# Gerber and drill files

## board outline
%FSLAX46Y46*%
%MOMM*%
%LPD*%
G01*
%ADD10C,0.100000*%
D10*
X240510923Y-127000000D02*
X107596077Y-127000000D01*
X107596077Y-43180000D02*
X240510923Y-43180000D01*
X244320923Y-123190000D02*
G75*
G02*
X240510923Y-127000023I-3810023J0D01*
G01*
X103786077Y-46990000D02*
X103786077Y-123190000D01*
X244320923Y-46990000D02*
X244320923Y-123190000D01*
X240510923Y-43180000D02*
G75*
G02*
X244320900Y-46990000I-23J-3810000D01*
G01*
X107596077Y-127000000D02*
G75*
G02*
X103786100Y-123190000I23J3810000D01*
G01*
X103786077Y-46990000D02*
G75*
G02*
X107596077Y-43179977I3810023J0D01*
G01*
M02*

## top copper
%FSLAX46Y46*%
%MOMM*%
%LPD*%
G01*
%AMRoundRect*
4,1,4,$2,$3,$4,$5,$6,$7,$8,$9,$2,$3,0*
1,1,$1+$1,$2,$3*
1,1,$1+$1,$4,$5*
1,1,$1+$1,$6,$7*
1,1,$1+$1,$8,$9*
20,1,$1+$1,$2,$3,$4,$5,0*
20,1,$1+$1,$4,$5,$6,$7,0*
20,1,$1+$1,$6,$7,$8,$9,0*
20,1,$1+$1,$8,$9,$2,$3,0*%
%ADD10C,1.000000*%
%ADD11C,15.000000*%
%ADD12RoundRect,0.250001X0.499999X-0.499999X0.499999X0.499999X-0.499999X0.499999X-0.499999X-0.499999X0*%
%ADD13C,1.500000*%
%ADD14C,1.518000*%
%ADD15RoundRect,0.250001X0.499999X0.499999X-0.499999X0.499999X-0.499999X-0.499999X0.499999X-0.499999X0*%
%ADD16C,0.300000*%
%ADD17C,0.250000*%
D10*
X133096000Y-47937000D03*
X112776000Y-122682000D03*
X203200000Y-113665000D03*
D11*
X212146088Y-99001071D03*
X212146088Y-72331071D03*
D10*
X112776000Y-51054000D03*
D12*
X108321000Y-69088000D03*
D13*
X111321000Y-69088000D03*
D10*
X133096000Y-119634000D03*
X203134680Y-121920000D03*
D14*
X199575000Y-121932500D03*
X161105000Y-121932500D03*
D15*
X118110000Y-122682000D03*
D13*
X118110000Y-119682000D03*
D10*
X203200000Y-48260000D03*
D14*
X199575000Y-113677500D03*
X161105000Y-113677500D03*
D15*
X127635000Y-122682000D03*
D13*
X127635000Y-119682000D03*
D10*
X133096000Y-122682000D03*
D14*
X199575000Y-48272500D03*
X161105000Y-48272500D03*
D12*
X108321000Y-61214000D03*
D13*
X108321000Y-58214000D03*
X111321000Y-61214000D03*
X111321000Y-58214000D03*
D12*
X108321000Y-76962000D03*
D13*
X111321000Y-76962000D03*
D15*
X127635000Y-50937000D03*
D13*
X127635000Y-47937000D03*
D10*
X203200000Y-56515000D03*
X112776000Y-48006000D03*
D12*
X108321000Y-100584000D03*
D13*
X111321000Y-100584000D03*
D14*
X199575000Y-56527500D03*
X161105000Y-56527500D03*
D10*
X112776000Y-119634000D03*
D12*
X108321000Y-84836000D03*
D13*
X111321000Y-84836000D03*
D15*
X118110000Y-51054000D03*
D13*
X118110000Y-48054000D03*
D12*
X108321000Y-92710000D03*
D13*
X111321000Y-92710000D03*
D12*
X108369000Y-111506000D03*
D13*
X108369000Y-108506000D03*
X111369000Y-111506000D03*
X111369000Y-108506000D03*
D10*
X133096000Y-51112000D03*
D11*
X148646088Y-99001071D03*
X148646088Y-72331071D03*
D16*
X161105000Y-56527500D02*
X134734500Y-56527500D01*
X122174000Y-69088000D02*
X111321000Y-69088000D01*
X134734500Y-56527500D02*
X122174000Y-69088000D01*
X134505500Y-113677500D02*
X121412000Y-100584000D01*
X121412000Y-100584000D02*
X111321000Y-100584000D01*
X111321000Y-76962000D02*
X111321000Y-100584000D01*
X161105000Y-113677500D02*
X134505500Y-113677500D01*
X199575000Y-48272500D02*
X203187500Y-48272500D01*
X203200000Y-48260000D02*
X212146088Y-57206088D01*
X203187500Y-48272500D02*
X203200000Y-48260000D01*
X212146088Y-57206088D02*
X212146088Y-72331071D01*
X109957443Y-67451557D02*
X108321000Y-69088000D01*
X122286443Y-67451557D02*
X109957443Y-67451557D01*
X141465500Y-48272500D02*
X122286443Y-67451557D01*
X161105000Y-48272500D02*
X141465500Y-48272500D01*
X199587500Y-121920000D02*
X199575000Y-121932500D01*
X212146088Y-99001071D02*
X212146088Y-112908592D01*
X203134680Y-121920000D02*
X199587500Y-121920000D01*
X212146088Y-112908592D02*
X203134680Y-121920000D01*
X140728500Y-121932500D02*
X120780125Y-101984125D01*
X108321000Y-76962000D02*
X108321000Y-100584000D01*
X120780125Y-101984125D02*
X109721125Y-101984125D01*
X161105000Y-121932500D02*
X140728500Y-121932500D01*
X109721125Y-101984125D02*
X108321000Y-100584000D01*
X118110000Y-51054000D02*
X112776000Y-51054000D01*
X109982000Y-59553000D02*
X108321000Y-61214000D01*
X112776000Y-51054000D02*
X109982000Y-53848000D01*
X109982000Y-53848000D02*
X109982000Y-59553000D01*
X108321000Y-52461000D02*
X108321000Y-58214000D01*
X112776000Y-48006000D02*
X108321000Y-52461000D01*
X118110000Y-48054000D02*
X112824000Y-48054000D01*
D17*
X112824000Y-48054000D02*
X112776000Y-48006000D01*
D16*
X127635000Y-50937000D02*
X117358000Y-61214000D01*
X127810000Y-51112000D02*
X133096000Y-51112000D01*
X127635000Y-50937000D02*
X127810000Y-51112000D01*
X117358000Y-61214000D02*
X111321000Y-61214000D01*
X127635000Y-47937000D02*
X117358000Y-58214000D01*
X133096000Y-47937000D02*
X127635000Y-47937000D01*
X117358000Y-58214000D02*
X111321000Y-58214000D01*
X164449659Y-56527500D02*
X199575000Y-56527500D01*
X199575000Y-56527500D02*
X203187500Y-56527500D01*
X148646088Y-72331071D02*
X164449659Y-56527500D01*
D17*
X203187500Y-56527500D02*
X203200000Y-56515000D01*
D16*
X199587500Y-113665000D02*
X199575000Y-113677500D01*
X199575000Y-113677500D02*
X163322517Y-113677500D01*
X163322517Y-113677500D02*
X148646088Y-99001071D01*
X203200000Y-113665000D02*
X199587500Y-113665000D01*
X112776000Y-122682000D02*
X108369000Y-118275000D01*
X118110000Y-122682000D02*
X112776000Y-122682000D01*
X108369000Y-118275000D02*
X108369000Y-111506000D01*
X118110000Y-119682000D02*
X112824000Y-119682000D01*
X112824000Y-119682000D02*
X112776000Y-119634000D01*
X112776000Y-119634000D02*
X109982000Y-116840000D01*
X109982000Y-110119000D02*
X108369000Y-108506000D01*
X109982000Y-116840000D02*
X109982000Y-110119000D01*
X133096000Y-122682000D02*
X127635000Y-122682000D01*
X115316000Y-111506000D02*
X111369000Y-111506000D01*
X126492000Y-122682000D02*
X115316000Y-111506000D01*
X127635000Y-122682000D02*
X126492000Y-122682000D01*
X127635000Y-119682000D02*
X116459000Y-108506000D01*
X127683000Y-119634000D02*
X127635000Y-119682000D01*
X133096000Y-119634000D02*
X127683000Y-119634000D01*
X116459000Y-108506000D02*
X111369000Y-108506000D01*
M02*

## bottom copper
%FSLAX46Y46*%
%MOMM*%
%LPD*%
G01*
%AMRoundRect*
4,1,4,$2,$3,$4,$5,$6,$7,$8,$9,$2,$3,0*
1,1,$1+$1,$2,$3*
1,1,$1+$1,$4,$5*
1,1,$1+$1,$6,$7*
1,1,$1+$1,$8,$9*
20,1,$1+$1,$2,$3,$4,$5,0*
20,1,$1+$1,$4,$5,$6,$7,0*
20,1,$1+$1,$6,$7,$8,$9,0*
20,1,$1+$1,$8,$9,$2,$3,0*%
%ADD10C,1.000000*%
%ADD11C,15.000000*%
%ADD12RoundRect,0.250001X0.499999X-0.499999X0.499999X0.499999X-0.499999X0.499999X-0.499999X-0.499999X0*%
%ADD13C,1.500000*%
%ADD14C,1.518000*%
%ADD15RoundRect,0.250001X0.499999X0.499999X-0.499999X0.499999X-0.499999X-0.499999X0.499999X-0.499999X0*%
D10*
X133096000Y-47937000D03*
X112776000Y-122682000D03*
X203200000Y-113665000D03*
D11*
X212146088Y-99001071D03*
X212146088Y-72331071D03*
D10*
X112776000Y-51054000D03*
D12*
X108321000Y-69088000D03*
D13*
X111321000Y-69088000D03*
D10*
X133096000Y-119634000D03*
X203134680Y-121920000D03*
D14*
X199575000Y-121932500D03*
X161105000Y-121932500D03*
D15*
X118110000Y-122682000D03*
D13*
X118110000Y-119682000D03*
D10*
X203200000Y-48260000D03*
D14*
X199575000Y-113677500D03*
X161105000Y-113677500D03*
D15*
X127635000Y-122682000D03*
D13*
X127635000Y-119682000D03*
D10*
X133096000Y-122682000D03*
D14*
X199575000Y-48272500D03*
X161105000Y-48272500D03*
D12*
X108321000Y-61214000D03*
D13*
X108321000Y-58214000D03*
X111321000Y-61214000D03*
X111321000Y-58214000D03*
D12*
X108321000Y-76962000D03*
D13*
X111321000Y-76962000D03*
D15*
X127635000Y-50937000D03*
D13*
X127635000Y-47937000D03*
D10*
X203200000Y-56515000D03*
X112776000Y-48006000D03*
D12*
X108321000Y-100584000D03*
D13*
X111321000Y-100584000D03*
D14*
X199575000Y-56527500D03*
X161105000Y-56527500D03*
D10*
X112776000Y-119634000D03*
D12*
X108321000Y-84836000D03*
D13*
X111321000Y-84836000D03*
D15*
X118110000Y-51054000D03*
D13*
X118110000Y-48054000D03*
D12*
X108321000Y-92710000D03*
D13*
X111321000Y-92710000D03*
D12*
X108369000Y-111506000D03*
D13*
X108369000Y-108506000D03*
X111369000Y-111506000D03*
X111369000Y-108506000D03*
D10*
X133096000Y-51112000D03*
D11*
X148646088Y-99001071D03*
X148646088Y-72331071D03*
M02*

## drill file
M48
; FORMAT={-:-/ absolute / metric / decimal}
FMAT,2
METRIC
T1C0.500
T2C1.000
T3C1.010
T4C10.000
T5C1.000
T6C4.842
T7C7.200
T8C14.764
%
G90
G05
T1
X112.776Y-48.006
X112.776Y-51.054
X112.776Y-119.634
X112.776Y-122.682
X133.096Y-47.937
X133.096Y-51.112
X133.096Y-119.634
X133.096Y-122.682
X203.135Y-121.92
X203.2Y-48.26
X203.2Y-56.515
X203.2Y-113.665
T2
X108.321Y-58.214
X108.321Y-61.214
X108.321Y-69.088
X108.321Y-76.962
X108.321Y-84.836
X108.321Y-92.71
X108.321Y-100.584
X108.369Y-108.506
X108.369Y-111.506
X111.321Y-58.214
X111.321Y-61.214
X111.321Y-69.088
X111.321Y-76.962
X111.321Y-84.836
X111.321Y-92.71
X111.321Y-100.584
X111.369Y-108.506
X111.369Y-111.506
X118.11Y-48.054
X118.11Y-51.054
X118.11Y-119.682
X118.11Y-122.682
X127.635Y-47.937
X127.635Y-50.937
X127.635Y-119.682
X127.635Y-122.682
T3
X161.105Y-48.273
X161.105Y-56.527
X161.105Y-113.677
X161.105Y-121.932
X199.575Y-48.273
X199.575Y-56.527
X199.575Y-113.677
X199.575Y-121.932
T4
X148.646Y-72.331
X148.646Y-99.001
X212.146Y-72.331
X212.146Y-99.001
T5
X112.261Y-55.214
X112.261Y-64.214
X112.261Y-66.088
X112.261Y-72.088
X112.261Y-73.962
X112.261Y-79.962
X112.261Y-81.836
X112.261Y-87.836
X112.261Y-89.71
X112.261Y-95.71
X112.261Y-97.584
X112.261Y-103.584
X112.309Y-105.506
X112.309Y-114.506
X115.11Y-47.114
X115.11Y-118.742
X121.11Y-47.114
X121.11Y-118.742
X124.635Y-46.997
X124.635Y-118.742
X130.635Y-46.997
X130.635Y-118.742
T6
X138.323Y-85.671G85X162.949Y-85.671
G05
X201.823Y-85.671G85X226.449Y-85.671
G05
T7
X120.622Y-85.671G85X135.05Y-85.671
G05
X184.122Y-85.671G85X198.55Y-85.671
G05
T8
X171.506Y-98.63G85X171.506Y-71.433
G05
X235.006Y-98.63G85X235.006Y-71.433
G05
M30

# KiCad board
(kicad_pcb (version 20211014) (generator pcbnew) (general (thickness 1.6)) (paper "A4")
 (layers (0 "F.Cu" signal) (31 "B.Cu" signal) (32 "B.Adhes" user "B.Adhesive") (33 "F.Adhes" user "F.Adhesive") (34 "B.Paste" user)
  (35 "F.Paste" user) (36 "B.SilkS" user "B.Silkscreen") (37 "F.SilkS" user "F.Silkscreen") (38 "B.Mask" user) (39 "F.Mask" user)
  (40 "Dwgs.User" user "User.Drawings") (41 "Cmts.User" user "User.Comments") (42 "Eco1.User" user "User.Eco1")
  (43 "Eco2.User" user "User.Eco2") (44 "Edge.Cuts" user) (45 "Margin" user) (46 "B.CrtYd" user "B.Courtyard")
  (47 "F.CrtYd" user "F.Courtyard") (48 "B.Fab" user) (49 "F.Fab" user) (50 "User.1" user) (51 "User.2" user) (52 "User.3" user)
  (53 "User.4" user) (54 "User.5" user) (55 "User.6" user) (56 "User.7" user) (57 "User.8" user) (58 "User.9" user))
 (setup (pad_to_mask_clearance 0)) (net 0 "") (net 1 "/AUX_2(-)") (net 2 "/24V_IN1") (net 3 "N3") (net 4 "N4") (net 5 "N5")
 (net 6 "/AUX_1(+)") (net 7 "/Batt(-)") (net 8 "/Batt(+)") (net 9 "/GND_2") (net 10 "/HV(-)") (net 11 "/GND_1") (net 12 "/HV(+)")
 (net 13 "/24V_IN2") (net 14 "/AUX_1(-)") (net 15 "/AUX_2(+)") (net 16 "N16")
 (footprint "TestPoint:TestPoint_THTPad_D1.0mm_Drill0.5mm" (layer "F.Cu") (at 133.096 47.937)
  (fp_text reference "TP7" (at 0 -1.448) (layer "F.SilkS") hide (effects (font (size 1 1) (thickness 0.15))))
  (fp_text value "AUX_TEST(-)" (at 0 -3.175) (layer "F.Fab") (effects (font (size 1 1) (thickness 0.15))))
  (pad "1" thru_hole circle (at 0 0) (size 1 1) (drill 0.5) (layers *.Cu *.Mask) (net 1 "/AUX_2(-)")))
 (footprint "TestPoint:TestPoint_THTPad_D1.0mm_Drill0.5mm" (layer "F.Cu") (at 112.776 122.682)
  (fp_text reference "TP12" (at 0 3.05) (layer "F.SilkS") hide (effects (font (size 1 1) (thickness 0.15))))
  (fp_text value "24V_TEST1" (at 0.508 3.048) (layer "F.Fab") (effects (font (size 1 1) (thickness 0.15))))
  (pad "1" thru_hole circle (at 0 0) (size 1 1) (drill 0.5) (layers *.Cu *.Mask) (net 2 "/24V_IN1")))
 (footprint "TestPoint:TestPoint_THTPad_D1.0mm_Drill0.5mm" (layer "F.Cu") (at 203.2 113.665)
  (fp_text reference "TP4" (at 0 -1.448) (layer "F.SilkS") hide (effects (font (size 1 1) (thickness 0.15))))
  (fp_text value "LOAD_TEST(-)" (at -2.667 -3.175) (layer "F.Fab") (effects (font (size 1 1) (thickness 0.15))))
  (pad "1" thru_hole circle (at 0 0) (size 1 1) (drill 0.5) (layers *.Cu *.Mask) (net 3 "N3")))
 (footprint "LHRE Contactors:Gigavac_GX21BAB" (layer "F.Cu") (at 182.738388 125.790071 90)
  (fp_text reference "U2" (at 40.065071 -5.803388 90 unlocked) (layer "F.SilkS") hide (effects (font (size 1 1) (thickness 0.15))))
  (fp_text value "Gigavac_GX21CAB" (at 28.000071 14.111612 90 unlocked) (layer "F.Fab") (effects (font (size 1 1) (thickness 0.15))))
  (pad "" np_thru_hole oval (at 40.119 31.3977 90) (size 4.84155 29.467172) (drill oval 4.84155 29.467172) (layers F&B.Cu *.Mask))
  (pad "" np_thru_hole oval (at 40.759 52.2677 90) (size 41.9608 14.76375) (drill oval 41.9608 14.76375) (layers F&B.Cu *.Mask))
  (pad "" np_thru_hole oval (at 40.119 8.5977 90) (size 7.2 21.6281) (drill oval 7.2 21.6281) (layers F&B.Cu *.Mask))
  (pad "1" thru_hole circle (at 26.789 29.4077 90) (size 15 15) (drill 10) (layers *.Cu *.Mask) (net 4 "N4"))
  (pad "2" thru_hole circle (at 53.459 29.4077 90) (size 15 15) (drill 10) (layers *.Cu *.Mask) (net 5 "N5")))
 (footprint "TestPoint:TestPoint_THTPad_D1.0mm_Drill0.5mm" (layer "F.Cu") (at 112.776 51.054)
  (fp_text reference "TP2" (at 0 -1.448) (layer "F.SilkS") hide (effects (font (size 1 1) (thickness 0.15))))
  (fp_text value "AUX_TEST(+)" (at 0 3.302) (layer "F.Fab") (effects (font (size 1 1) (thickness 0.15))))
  (pad "1" thru_hole circle (at 0 0) (size 1 1) (drill 0.5) (layers *.Cu *.Mask) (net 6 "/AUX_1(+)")))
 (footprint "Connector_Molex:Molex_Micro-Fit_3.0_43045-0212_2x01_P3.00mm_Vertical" (layer "F.Cu") (at 108.321 69.088 90)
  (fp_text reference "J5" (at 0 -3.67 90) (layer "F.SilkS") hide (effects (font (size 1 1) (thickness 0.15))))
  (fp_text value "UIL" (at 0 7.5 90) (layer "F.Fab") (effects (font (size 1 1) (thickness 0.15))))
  (pad "" np_thru_hole circle (at 3 3.94 90) (size 1 1) (drill 1) (layers *.Cu *.Mask))
  (pad "" np_thru_hole circle (at -3 3.94 90) (size 1 1) (drill 1) (layers *.Cu *.Mask))
  (pad "1" thru_hole roundrect (at 0 0 90) (size 1.5 1.5) (drill 1) (layers *.Cu *.Mask) (roundrect_rratio 0.166667) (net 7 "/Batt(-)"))
  (pad "2" thru_hole circle (at 0 3 90) (size 1.5 1.5) (drill 1) (layers *.Cu *.Mask) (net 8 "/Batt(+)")))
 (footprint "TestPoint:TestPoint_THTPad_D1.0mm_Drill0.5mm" (layer "F.Cu") (at 133.096 119.634)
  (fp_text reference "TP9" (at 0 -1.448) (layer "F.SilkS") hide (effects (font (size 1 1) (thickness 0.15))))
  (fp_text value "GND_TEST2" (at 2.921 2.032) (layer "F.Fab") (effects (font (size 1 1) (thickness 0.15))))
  (pad "1" thru_hole circle (at 0 0) (size 1 1) (drill 0.5) (layers *.Cu *.Mask) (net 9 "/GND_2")))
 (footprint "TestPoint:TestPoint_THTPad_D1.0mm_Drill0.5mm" (layer "F.Cu") (at 203.13468 121.92)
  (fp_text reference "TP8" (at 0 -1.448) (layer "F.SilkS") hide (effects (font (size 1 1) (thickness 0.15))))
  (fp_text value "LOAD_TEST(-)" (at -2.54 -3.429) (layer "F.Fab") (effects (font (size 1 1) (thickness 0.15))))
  (pad "1" thru_hole circle (at 0 0) (size 1 1) (drill 0.5) (layers *.Cu *.Mask) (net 4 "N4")))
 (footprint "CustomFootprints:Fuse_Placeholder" (layer "F.Cu") (at 180.44 129.1225 180)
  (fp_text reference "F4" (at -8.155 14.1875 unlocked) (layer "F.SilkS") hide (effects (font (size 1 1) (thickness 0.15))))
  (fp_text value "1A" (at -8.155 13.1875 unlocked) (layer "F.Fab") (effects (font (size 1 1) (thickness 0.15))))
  (pad "1" thru_hole circle (at -19.135 7.19 180) (size 1.518 1.518) (drill 1.01) (layers *.Cu *.Mask) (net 4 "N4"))
  (pad "2" thru_hole circle (at 19.335 7.19 180) (size 1.518 1.518) (drill 1.01) (layers *.Cu *.Mask) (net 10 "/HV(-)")))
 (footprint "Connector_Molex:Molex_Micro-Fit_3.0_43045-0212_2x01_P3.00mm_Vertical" (layer "F.Cu") (at 118.11 122.682 180)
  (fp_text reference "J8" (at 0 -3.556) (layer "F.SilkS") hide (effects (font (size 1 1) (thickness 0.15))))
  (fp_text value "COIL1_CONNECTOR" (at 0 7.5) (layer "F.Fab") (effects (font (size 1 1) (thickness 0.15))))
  (pad "" np_thru_hole circle (at -3 3.94 180) (size 1 1) (drill 1) (layers *.Cu *.Mask))
  (pad "" np_thru_hole circle (at 3 3.94 180) (size 1 1) (drill 1) (layers *.Cu *.Mask))
  (pad "1" thru_hole roundrect (at 0 0 180) (size 1.5 1.5) (drill 1) (layers *.Cu *.Mask) (roundrect_rratio 0.166667) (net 2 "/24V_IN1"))
  (pad "2" thru_hole circle (at 0 3 180) (size 1.5 1.5) (drill 1) (layers *.Cu *.Mask) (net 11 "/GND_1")))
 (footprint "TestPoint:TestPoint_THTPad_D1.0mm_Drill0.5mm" (layer "F.Cu") (at 203.2 48.26)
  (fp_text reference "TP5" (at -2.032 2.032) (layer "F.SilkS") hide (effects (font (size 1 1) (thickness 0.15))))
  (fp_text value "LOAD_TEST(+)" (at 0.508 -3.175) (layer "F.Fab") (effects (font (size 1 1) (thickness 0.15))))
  (pad "1" thru_hole circle (at 0 0) (size 1 1) (drill 0.5) (layers *.Cu *.Mask) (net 5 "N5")))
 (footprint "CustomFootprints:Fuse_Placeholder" (layer "F.Cu") (at 180.44 120.8675 180)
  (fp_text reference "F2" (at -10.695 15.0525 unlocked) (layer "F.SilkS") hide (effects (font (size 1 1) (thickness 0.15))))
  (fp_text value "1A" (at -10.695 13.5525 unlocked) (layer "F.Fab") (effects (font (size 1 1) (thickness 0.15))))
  (pad "1" thru_hole circle (at -19.135 7.19 180) (size 1.518 1.518) (drill 1.01) (layers *.Cu *.Mask) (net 3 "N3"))
  (pad "2" thru_hole circle (at 19.335 7.19 180) (size 1.518 1.518) (drill 1.01) (layers *.Cu *.Mask) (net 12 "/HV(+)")))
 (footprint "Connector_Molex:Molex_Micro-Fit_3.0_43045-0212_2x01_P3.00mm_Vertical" (layer "F.Cu") (at 127.635 122.682 180)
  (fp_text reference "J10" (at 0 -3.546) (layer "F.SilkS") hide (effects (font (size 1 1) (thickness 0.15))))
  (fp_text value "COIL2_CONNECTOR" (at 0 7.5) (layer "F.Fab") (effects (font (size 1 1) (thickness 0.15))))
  (pad "" np_thru_hole circle (at -3 3.94 180) (size 1 1) (drill 1) (layers *.Cu *.Mask))
  (pad "" np_thru_hole circle (at 3 3.94 180) (size 1 1) (drill 1) (layers *.Cu *.Mask))
  (pad "1" thru_hole roundrect (at 0 0 180) (size 1.5 1.5) (drill 1) (layers *.Cu *.Mask) (roundrect_rratio 0.166667) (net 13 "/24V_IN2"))
  (pad "2" thru_hole circle (at 0 3 180) (size 1.5 1.5) (drill 1) (layers *.Cu *.Mask) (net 9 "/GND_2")))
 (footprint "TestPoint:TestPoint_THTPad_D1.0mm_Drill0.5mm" (layer "F.Cu") (at 133.096 122.682)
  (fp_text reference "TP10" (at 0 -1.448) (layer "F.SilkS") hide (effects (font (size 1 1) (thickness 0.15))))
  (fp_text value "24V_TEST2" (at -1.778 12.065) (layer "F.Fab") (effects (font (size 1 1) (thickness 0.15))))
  (pad "1" thru_hole circle (at 0 0) (size 1 1) (drill 0.5) (layers *.Cu *.Mask) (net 13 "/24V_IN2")))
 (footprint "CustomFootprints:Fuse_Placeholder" (layer "F.Cu") (at 180.44 55.4625 180)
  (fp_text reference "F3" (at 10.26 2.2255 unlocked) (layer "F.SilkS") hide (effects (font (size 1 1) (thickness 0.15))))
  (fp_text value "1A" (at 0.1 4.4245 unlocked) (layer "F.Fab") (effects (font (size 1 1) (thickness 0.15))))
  (pad "1" thru_hole circle (at -19.135 7.19 180) (size 1.518 1.518) (drill 1.01) (layers *.Cu *.Mask) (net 5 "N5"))
  (pad "2" thru_hole circle (at 19.335 7.19 180) (size 1.518 1.518) (drill 1.01) (layers *.Cu *.Mask) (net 7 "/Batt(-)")))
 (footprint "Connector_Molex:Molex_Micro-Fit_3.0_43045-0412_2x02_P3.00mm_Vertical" (layer "F.Cu") (at 108.321 61.214 90)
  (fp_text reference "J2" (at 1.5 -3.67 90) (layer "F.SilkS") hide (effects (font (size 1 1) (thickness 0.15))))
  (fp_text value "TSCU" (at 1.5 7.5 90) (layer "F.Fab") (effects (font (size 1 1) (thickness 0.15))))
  (pad "" np_thru_hole circle (at -3 3.94 90) (size 1 1) (drill 1) (layers *.Cu *.Mask))
  (pad "" np_thru_hole circle (at 6 3.94 90) (size 1 1) (drill 1) (layers *.Cu *.Mask))
  (pad "1" thru_hole roundrect (at 0 0 90) (size 1.5 1.5) (drill 1) (layers *.Cu *.Mask) (roundrect_rratio 0.166667) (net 6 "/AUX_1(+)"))
  (pad "2" thru_hole circle (at 3 0 90) (size 1.5 1.5) (drill 1) (layers *.Cu *.Mask) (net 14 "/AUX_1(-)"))
  (pad "3" thru_hole circle (at 0 3 90) (size 1.5 1.5) (drill 1) (layers *.Cu *.Mask) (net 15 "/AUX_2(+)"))
  (pad "4" thru_hole circle (at 3 3 90) (size 1.5 1.5) (drill 1) (layers *.Cu *.Mask) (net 1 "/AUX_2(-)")))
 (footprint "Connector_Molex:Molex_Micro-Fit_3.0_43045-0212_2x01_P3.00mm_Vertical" (layer "F.Cu") (at 108.321 76.962 90)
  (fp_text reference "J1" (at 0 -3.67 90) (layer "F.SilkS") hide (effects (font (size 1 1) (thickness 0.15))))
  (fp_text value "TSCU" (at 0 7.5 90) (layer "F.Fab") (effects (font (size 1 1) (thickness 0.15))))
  (pad "" np_thru_hole circle (at 3 3.94 90) (size 1 1) (drill 1) (layers *.Cu *.Mask))
  (pad "" np_thru_hole circle (at -3 3.94 90) (size 1 1) (drill 1) (layers *.Cu *.Mask))
  (pad "1" thru_hole roundrect (at 0 0 90) (size 1.5 1.5) (drill 1) (layers *.Cu *.Mask) (roundrect_rratio 0.166667) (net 10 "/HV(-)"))
  (pad "2" thru_hole circle (at 0 3 90) (size 1.5 1.5) (drill 1) (layers *.Cu *.Mask) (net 12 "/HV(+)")))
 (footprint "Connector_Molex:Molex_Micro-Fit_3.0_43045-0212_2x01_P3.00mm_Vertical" (layer "F.Cu") (at 127.635 50.937 180)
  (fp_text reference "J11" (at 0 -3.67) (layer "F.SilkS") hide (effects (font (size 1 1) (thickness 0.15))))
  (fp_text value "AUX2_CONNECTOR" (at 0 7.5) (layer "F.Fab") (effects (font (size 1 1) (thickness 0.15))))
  (pad "" np_thru_hole circle (at 3 3.94 180) (size 1 1) (drill 1) (layers *.Cu *.Mask))
  (pad "" np_thru_hole circle (at -3 3.94 180) (size 1 1) (drill 1) (layers *.Cu *.Mask))
  (pad "1" thru_hole roundrect (at 0 0 180) (size 1.5 1.5) (drill 1) (layers *.Cu *.Mask) (roundrect_rratio 0.166667) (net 15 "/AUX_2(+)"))
  (pad "2" thru_hole circle (at 0 3 180) (size 1.5 1.5) (drill 1) (layers *.Cu *.Mask) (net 1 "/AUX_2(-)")))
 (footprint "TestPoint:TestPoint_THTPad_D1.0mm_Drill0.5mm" (layer "F.Cu") (at 203.2 56.515)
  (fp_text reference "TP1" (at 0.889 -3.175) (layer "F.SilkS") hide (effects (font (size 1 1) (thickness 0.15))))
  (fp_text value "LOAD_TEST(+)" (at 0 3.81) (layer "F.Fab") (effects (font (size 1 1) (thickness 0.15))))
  (pad "1" thru_hole circle (at 0 0) (size 1 1) (drill 0.5) (layers *.Cu *.Mask) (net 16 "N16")))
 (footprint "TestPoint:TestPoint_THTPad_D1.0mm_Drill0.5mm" (layer "F.Cu") (at 112.776 48.006)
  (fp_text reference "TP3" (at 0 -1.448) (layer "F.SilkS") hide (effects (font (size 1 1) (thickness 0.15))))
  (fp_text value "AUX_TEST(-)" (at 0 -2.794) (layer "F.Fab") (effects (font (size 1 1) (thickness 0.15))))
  (pad "1" thru_hole circle (at 0 0) (size 1 1) (drill 0.5) (layers *.Cu *.Mask) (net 14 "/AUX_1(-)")))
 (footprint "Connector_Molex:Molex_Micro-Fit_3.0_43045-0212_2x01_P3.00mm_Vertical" (layer "F.Cu") (at 108.321 100.584 90)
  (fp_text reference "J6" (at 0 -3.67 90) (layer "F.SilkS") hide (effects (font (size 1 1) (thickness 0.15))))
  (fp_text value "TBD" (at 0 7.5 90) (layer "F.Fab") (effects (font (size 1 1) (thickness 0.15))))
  (pad "" np_thru_hole circle (at 3 3.94 90) (size 1 1) (drill 1) (layers *.Cu *.Mask))
  (pad "" np_thru_hole circle (at -3 3.94 90) (size 1 1) (drill 1) (layers *.Cu *.Mask))
  (pad "1" thru_hole roundrect (at 0 0 90) (size 1.5 1.5) (drill 1) (layers *.Cu *.Mask) (roundrect_rratio 0.166667) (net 10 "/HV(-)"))
  (pad "2" thru_hole circle (at 0 3 90) (size 1.5 1.5) (drill 1) (layers *.Cu *.Mask) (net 12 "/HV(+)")))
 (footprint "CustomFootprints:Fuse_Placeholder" (layer "F.Cu") (at 180.44 63.7175 180)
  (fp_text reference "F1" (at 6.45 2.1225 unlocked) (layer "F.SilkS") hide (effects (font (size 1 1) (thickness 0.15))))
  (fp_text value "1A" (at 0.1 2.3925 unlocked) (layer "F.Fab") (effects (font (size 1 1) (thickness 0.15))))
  (pad "1" thru_hole circle (at -19.135 7.19 180) (size 1.518 1.518) (drill 1.01) (layers *.Cu *.Mask) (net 16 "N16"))
  (pad "2" thru_hole circle (at 19.335 7.19 180) (size 1.518 1.518) (drill 1.01) (layers *.Cu *.Mask) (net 8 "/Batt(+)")))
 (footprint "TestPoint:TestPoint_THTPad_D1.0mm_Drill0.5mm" (layer "F.Cu") (at 112.776 119.634)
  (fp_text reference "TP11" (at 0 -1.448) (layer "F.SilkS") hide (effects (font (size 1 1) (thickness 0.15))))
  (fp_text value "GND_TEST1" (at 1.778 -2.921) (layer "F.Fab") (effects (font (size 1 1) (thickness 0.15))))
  (pad "1" thru_hole circle (at 0 0) (size 1 1) (drill 0.5) (layers *.Cu *.Mask) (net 11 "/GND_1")))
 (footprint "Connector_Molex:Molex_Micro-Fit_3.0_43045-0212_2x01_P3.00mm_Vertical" (layer "F.Cu") (at 108.321 84.836 90)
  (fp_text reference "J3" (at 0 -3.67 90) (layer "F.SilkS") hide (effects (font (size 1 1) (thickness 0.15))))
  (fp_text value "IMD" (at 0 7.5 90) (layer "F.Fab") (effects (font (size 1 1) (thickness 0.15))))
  (pad "" np_thru_hole circle (at 3 3.94 90) (size 1 1) (drill 1) (layers *.Cu *.Mask))
  (pad "" np_thru_hole circle (at -3 3.94 90) (size 1 1) (drill 1) (layers *.Cu *.Mask))
  (pad "1" thru_hole roundrect (at 0 0 90) (size 1.5 1.5) (drill 1) (layers *.Cu *.Mask) (roundrect_rratio 0.166667) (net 10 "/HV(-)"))
  (pad "2" thru_hole circle (at 0 3 90) (size 1.5 1.5) (drill 1) (layers *.Cu *.Mask) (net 12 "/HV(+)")))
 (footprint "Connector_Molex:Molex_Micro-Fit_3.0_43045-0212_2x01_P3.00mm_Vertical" (layer "F.Cu") (at 118.11 51.054 180)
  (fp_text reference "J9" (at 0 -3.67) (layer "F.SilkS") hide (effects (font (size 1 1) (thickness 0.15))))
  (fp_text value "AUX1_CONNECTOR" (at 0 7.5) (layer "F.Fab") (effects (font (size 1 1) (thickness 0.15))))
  (pad "" np_thru_hole circle (at 3 3.94 180) (size 1 1) (drill 1) (layers *.Cu *.Mask))
  (pad "" np_thru_hole circle (at -3 3.94 180) (size 1 1) (drill 1) (layers *.Cu *.Mask))
  (pad "1" thru_hole roundrect (at 0 0 180) (size 1.5 1.5) (drill 1) (layers *.Cu *.Mask) (roundrect_rratio 0.166667) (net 6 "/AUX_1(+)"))
  (pad "2" thru_hole circle (at 0 3 180) (size 1.5 1.5) (drill 1) (layers *.Cu *.Mask) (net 14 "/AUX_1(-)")))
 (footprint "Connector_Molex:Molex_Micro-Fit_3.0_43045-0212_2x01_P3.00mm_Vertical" (layer "F.Cu") (at 108.321 92.71 90)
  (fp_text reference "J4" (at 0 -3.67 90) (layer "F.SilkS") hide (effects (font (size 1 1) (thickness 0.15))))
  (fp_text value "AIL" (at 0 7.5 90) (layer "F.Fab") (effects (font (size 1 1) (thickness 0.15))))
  (pad "" np_thru_hole circle (at 3 3.94 90) (size 1 1) (drill 1) (layers *.Cu *.Mask))
  (pad "" np_thru_hole circle (at -3 3.94 90) (size 1 1) (drill 1) (layers *.Cu *.Mask))
  (pad "1" thru_hole roundrect (at 0 0 90) (size 1.5 1.5) (drill 1) (layers *.Cu *.Mask) (roundrect_rratio 0.166667) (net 10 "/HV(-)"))
  (pad "2" thru_hole circle (at 0 3 90) (size 1.5 1.5) (drill 1) (layers *.Cu *.Mask) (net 12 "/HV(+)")))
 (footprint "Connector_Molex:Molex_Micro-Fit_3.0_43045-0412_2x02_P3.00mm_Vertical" (layer "F.Cu") (at 108.369 111.506 90)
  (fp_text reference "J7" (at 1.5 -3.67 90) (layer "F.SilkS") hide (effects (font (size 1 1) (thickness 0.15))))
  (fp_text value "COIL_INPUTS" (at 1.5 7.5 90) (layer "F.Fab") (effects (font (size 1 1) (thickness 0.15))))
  (pad "" np_thru_hole circle (at 6 3.94 90) (size 1 1) (drill 1) (layers *.Cu *.Mask))
  (pad "" np_thru_hole circle (at -3 3.94 90) (size 1 1) (drill 1) (layers *.Cu *.Mask))
  (pad "1" thru_hole roundrect (at 0 0 90) (size 1.5 1.5) (drill 1) (layers *.Cu *.Mask) (roundrect_rratio 0.166667) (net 2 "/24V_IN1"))
  (pad "2" thru_hole circle (at 3 0 90) (size 1.5 1.5) (drill 1) (layers *.Cu *.Mask) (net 11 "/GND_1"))
  (pad "3" thru_hole circle (at 0 3 90) (size 1.5 1.5) (drill 1) (layers *.Cu *.Mask) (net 13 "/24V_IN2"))
  (pad "4" thru_hole circle (at 3 3 90) (size 1.5 1.5) (drill 1) (layers *.Cu *.Mask) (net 9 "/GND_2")))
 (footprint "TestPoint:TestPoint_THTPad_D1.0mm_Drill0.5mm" (layer "F.Cu") (at 133.096 51.112)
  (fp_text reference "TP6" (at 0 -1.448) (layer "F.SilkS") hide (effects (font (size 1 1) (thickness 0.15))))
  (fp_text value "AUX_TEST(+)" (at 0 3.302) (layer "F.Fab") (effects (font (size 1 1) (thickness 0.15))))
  (pad "1" thru_hole circle (at 0 0) (size 1 1) (drill 0.5) (layers *.Cu *.Mask) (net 15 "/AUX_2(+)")))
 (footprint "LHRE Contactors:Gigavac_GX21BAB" (layer "F.Cu") (at 119.238388 125.790071 90)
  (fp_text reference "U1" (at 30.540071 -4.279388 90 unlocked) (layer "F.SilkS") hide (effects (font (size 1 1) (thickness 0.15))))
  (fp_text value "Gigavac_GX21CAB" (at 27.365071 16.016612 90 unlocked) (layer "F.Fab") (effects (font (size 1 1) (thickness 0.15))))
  (pad "" np_thru_hole oval (at 40.119 8.5977 90) (size 7.2 21.6281) (drill oval 7.2 21.6281) (layers F&B.Cu *.Mask))
  (pad "" np_thru_hole oval (at 40.119 31.3977 90) (size 4.84155 29.467172) (drill oval 4.84155 29.467172) (layers F&B.Cu *.Mask))
  (pad "" np_thru_hole oval (at 40.759 52.2677 90) (size 41.9608 14.76375) (drill oval 41.9608 14.76375) (layers F&B.Cu *.Mask))
  (pad "1" thru_hole circle (at 26.789 29.4077 90) (size 15 15) (drill 10) (layers *.Cu *.Mask) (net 3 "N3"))
  (pad "2" thru_hole circle (at 53.459 29.4077 90) (size 15 15) (drill 10) (layers *.Cu *.Mask) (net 16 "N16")))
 (gr_line (start 240.510923 127) (end 107.596077 127) (layer "Edge.Cuts") (width 0.1))
 (gr_line (start 107.596077 43.18) (end 240.510923 43.18) (layer "Edge.Cuts") (width 0.1))
 (gr_arc (start 244.320923 123.19) (mid 243.205 125.884077) (end 240.510923 127) (layer "Edge.Cuts") (width 0.1))
 (gr_line (start 103.786077 46.99) (end 103.786077 123.19) (layer "Edge.Cuts") (width 0.1))
 (gr_line (start 244.320923 46.99) (end 244.320923 123.19) (layer "Edge.Cuts") (width 0.1))
 (gr_arc (start 240.510923 43.18) (mid 243.205 44.295923) (end 244.320923 46.99) (layer "Edge.Cuts") (width 0.1))
 (gr_arc (start 107.596077 127) (mid 104.902 125.884077) (end 103.786077 123.19) (layer "Edge.Cuts") (width 0.1))
 (gr_arc (start 103.786077 46.99) (mid 104.902 44.295923) (end 107.596077 43.18) (layer "Edge.Cuts") (width 0.1))
 (segment (start 161.105 56.5275) (end 134.7345 56.5275) (width 0.3) (layer "F.Cu") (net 8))
 (segment (start 122.174 69.088) (end 111.321 69.088) (width 0.3) (layer "F.Cu") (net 8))
 (segment (start 134.7345 56.5275) (end 122.174 69.088) (width 0.3) (layer "F.Cu") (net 8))
 (segment (start 134.5055 113.6775) (end 121.412 100.584) (width 0.3) (layer "F.Cu") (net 12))
 (segment (start 121.412 100.584) (end 111.321 100.584) (width 0.3) (layer "F.Cu") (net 12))
 (segment (start 111.321 76.962) (end 111.321 100.584) (width 0.3) (layer "F.Cu") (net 12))
 (segment (start 161.105 113.6775) (end 134.5055 113.6775) (width 0.3) (layer "F.Cu") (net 12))
 (segment (start 199.575 48.2725) (end 203.1875 48.2725) (width 0.3) (layer "F.Cu") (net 5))
 (segment (start 203.2 48.26) (end 212.146088 57.206088) (width 0.3) (layer "F.Cu") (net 5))
 (segment (start 203.1875 48.2725) (end 203.2 48.26) (width 0.3) (layer "F.Cu") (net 5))
 (segment (start 212.146088 57.206088) (end 212.146088 72.331071) (width 0.3) (layer "F.Cu") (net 5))
 (segment (start 109.957443 67.451557) (end 108.321 69.088) (width 0.3) (layer "F.Cu") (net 7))
 (segment (start 122.286443 67.451557) (end 109.957443 67.451557) (width 0.3) (layer "F.Cu") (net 7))
 (segment (start 141.4655 48.2725) (end 122.286443 67.451557) (width 0.3) (layer "F.Cu") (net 7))
 (segment (start 161.105 48.2725) (end 141.4655 48.2725) (width 0.3) (layer "F.Cu") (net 7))
 (segment (start 199.5875 121.92) (end 199.575 121.9325) (width 0.3) (layer "F.Cu") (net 4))
 (segment (start 212.146088 99.001071) (end 212.146088 112.908592) (width 0.3) (layer "F.Cu") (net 4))
 (segment (start 203.13468 121.92) (end 199.5875 121.92) (width 0.3) (layer "F.Cu") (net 4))
 (segment (start 212.146088 112.908592) (end 203.13468 121.92) (width 0.3) (layer "F.Cu") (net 4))
 (segment (start 140.7285 121.9325) (end 120.780125 101.984125) (width 0.3) (layer "F.Cu") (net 10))
 (segment (start 108.321 76.962) (end 108.321 100.584) (width 0.3) (layer "F.Cu") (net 10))
 (segment (start 120.780125 101.984125) (end 109.721125 101.984125) (width 0.3) (layer "F.Cu") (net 10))
 (segment (start 161.105 121.9325) (end 140.7285 121.9325) (width 0.3) (layer "F.Cu") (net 10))
 (segment (start 109.721125 101.984125) (end 108.321 100.584) (width 0.3) (layer "F.Cu") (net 10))
 (segment (start 118.11 51.054) (end 112.776 51.054) (width 0.3) (layer "F.Cu") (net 6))
 (segment (start 109.982 59.553) (end 108.321 61.214) (width 0.3) (layer "F.Cu") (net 6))
 (segment (start 112.776 51.054) (end 109.982 53.848) (width 0.3) (layer "F.Cu") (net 6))
 (segment (start 109.982 53.848) (end 109.982 59.553) (width 0.3) (layer "F.Cu") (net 6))
 (segment (start 108.321 52.461) (end 108.321 58.214) (width 0.3) (layer "F.Cu") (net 14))
 (segment (start 112.776 48.006) (end 108.321 52.461) (width 0.3) (layer "F.Cu") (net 14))
 (segment (start 118.11 48.054) (end 112.824 48.054) (width 0.3) (layer "F.Cu") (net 14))
 (segment (start 112.824 48.054) (end 112.776 48.006) (width 0.25) (layer "F.Cu") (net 14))
 (segment (start 127.635 50.937) (end 117.358 61.214) (width 0.3) (layer "F.Cu") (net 15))
 (segment (start 127.81 51.112) (end 133.096 51.112) (width 0.3) (layer "F.Cu") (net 15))
 (segment (start 127.635 50.937) (end 127.81 51.112) (width 0.3) (layer "F.Cu") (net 15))
 (segment (start 117.358 61.214) (end 111.321 61.214) (width 0.3) (layer "F.Cu") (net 15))
 (segment (start 127.635 47.937) (end 117.358 58.214) (width 0.3) (layer "F.Cu") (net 1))
 (segment (start 133.096 47.937) (end 127.635 47.937) (width 0.3) (layer "F.Cu") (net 1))
 (segment (start 117.358 58.214) (end 111.321 58.214) (width 0.3) (layer "F.Cu") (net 1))
 (segment (start 164.449659 56.5275) (end 199.575 56.5275) (width 0.3) (layer "F.Cu") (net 16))
 (segment (start 199.575 56.5275) (end 203.1875 56.5275) (width 0.3) (layer "F.Cu") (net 16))
 (segment (start 148.646088 72.331071) (end 164.449659 56.5275) (width 0.3) (layer "F.Cu") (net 16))
 (segment (start 203.1875 56.5275) (end 203.2 56.515) (width 0.25) (layer "F.Cu") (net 16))
 (segment (start 199.5875 113.665) (end 199.575 113.6775) (width 0.3) (layer "F.Cu") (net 3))
 (segment (start 199.575 113.6775) (end 163.322517 113.6775) (width 0.3) (layer "F.Cu") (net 3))
 (segment (start 163.322517 113.6775) (end 148.646088 99.001071) (width 0.3) (layer "F.Cu") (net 3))
 (segment (start 203.2 113.665) (end 199.5875 113.665) (width 0.3) (layer "F.Cu") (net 3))
 (segment (start 112.776 122.682) (end 108.369 118.275) (width 0.3) (layer "F.Cu") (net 2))
 (segment (start 118.11 122.682) (end 112.776 122.682) (width 0.3) (layer "F.Cu") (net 2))
 (segment (start 108.369 118.275) (end 108.369 111.506) (width 0.3) (layer "F.Cu") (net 2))
 (segment (start 118.11 119.682) (end 112.824 119.682) (width 0.3) (layer "F.Cu") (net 11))
 (segment (start 112.824 119.682) (end 112.776 119.634) (width 0.3) (layer "F.Cu") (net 11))
 (segment (start 112.776 119.634) (end 109.982 116.84) (width 0.3) (layer "F.Cu") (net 11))
 (segment (start 109.982 110.119) (end 108.369 108.506) (width 0.3) (layer "F.Cu") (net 11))
 (segment (start 109.982 116.84) (end 109.982 110.119) (width 0.3) (layer "F.Cu") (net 11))
 (segment (start 133.096 122.682) (end 127.635 122.682) (width 0.3) (layer "F.Cu") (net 13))
 (segment (start 115.316 111.506) (end 111.369 111.506) (width 0.3) (layer "F.Cu") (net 13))
 (segment (start 126.492 122.682) (end 115.316 111.506) (width 0.3) (layer "F.Cu") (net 13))
 (segment (start 127.635 122.682) (end 126.492 122.682) (width 0.3) (layer "F.Cu") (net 13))
 (segment (start 127.635 119.682) (end 116.459 108.506) (width 0.3) (layer "F.Cu") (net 9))
 (segment (start 127.683 119.634) (end 127.635 119.682) (width 0.3) (layer "F.Cu") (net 9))
 (segment (start 133.096 119.634) (end 127.683 119.634) (width 0.3) (layer "F.Cu") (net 9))
 (segment (start 116.459 108.506) (end 111.369 108.506) (width 0.3) (layer "F.Cu") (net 9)))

